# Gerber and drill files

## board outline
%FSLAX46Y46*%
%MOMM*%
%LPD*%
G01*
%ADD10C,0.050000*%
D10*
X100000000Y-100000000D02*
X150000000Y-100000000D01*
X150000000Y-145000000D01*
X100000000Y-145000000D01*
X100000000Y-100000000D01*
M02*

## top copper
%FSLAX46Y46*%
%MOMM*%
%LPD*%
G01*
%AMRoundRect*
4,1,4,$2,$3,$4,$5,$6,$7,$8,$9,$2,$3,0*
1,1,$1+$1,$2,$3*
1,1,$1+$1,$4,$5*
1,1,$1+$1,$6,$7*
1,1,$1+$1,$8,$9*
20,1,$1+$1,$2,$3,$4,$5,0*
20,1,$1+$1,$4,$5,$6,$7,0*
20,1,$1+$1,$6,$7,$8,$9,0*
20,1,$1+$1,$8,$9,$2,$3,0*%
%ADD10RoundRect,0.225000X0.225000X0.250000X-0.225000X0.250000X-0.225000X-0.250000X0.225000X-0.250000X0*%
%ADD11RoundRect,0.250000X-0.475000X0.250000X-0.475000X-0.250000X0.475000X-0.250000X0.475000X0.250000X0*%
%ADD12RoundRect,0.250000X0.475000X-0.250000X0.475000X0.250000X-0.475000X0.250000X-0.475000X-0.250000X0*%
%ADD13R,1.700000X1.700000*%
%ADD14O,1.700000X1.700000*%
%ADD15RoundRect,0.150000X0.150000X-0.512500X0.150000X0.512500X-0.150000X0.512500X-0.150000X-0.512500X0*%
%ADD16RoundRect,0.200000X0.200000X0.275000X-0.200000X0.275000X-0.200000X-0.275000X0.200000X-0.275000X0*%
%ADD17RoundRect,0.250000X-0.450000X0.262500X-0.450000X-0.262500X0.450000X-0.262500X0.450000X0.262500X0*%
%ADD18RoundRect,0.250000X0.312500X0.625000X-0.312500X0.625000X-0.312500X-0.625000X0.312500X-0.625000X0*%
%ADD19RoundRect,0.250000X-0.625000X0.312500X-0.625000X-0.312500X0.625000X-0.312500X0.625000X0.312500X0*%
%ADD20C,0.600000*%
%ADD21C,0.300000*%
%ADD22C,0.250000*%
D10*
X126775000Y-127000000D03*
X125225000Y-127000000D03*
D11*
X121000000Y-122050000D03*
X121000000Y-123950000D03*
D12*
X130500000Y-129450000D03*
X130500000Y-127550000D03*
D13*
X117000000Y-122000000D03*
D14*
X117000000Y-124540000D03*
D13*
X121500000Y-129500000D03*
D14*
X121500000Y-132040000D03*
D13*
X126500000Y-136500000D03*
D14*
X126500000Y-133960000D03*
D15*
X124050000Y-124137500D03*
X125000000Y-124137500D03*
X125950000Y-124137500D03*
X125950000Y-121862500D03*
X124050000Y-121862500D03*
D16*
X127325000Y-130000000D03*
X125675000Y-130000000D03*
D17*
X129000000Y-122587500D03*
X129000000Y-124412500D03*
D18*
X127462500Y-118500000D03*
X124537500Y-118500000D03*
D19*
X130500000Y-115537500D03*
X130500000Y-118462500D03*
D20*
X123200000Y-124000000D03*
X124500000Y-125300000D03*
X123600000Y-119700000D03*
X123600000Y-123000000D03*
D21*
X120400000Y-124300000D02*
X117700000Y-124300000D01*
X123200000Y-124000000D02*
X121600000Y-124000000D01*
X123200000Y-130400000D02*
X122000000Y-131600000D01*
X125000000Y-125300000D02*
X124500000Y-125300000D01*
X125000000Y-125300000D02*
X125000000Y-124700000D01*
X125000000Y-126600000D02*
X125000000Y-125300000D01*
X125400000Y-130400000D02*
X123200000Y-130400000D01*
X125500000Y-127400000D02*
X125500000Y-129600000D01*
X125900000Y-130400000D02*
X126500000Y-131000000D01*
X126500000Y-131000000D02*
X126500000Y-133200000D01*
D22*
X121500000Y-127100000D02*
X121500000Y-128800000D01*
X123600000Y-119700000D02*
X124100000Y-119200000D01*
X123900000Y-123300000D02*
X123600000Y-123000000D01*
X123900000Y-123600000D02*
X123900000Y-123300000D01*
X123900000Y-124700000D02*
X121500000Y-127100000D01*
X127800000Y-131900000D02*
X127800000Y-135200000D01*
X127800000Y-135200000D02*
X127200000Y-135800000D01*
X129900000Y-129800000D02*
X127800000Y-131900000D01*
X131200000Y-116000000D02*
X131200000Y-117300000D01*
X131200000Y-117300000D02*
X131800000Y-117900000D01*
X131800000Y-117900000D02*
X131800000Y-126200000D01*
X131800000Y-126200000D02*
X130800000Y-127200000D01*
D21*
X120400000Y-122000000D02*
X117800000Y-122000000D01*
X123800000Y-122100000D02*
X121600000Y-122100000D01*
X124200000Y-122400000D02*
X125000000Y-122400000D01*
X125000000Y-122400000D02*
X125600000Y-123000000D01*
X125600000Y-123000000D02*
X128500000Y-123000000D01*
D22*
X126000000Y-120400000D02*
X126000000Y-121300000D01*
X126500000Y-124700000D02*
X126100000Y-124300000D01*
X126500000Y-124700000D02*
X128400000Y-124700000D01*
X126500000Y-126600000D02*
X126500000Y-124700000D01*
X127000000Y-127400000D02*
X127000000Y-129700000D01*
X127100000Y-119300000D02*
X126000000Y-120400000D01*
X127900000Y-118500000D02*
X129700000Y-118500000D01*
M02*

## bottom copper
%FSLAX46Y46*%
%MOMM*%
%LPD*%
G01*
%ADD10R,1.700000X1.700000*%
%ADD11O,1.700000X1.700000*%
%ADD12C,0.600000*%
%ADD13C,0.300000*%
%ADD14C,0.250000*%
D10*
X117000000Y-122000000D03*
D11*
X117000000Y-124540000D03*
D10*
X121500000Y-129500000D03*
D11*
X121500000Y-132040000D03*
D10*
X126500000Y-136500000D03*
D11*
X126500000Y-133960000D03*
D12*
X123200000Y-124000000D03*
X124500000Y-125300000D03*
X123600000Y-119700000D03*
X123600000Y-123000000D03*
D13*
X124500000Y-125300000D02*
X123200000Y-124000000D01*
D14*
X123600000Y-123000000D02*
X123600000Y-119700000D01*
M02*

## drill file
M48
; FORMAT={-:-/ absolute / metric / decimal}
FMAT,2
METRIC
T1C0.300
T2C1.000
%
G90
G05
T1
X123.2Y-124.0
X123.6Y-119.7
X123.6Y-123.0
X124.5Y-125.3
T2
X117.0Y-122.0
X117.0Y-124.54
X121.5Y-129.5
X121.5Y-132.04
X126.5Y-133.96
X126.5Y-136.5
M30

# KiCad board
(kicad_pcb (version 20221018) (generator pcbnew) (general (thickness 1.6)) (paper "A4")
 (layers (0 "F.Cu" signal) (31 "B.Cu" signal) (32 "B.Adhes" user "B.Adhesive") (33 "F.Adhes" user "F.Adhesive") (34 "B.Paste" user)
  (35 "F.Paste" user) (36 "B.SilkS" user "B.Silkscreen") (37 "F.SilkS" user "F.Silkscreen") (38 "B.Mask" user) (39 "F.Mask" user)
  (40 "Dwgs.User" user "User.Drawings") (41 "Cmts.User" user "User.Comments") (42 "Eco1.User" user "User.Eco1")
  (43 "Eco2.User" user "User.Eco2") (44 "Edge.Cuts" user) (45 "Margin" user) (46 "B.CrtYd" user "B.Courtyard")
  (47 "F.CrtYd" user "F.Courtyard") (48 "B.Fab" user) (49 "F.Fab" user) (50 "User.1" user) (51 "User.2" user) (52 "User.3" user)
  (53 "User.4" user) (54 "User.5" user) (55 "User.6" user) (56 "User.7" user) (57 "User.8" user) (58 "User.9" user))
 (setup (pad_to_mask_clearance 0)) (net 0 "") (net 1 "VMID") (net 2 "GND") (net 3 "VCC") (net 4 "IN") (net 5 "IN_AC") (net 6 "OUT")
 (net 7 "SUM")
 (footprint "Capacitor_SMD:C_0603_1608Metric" (layer "F.Cu") (at 126 127 180)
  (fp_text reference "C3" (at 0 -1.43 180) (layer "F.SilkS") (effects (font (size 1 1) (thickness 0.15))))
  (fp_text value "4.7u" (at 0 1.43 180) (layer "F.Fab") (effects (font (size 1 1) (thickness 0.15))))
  (pad "1" smd roundrect (at -0.775 0 180) (size 0.9 0.95) (layers "F.Cu" "F.Paste" "F.Mask") (roundrect_rratio 0.25) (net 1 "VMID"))
  (pad "2" smd roundrect (at 0.775 0 180) (size 0.9 0.95) (layers "F.Cu" "F.Paste" "F.Mask") (roundrect_rratio 0.25) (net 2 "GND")))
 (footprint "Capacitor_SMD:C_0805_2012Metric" (layer "F.Cu") (at 121 123 -90)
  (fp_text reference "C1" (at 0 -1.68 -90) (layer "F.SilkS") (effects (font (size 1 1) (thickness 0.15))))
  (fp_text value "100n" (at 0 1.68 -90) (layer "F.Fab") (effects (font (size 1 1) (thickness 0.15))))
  (pad "1" smd roundrect (at -0.95 0 270) (size 1 1.45) (layers "F.Cu" "F.Paste" "F.Mask") (roundrect_rratio 0.25) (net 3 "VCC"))
  (pad "2" smd roundrect (at 0.95 0 270) (size 1 1.45) (layers "F.Cu" "F.Paste" "F.Mask") (roundrect_rratio 0.25) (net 2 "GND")))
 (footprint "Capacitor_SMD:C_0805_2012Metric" (layer "F.Cu") (at 130.5 128.5 90)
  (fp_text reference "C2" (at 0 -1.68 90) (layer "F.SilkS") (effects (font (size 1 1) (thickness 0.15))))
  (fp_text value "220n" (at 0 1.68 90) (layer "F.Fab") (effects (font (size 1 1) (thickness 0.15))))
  (pad "1" smd roundrect (at -0.95 0 90) (size 1 1.45) (layers "F.Cu" "F.Paste" "F.Mask") (roundrect_rratio 0.25) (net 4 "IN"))
  (pad "2" smd roundrect (at 0.95 0 90) (size 1 1.45) (layers "F.Cu" "F.Paste" "F.Mask") (roundrect_rratio 0.25) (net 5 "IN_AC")))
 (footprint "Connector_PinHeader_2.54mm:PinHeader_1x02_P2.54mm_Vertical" (layer "F.Cu") (at 117 122)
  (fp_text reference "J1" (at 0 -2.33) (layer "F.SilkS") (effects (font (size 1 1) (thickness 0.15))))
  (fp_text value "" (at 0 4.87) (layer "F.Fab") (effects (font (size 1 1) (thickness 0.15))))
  (pad "1" thru_hole rect (at 0 0) (size 1.7 1.7) (drill 1) (layers "*.Cu" "*.Mask") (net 3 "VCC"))
  (pad "2" thru_hole oval (at 0 2.54) (size 1.7 1.7) (drill 1) (layers "*.Cu" "*.Mask") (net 2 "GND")))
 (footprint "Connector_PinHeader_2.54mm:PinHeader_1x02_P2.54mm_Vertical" (layer "F.Cu") (at 121.5 129.5)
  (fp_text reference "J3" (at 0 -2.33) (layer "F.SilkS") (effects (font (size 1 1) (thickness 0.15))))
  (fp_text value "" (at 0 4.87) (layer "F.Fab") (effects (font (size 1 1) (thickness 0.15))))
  (pad "1" thru_hole rect (at 0 0) (size 1.7 1.7) (drill 1) (layers "*.Cu" "*.Mask") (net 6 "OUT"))
  (pad "2" thru_hole oval (at 0 2.54) (size 1.7 1.7) (drill 1) (layers "*.Cu" "*.Mask") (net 2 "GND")))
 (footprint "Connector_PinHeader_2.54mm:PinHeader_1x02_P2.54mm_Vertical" (layer "F.Cu") (at 126.5 136.5 180)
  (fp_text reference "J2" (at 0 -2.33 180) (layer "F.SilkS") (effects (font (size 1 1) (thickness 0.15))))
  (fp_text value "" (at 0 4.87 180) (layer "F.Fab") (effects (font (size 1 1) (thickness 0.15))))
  (pad "1" thru_hole rect (at 0 0 180) (size 1.7 1.7) (drill 1) (layers "*.Cu" "*.Mask") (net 4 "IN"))
  (pad "2" thru_hole oval (at 0 2.54 180) (size 1.7 1.7) (drill 1) (layers "*.Cu" "*.Mask") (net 2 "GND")))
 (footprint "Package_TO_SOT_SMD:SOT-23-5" (layer "F.Cu") (at 125 123 90)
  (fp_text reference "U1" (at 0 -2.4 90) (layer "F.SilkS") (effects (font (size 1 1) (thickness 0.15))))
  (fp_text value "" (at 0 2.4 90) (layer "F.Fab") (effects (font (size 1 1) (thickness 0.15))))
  (pad "1" smd roundrect (at -1.1375 -0.95 90) (size 1.325 0.6) (layers "F.Cu" "F.Paste" "F.Mask") (roundrect_rratio 0.25) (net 6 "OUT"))
  (pad "2" smd roundrect (at -1.1375 0 90) (size 1.325 0.6) (layers "F.Cu" "F.Paste" "F.Mask") (roundrect_rratio 0.25) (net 2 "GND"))
  (pad "3" smd roundrect (at -1.1375 0.95 90) (size 1.325 0.6) (layers "F.Cu" "F.Paste" "F.Mask") (roundrect_rratio 0.25) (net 1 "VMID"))
  (pad "4" smd roundrect (at 1.1375 0.95 90) (size 1.325 0.6) (layers "F.Cu" "F.Paste" "F.Mask") (roundrect_rratio 0.25) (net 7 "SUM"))
  (pad "5" smd roundrect (at 1.1375 -0.95 90) (size 1.325 0.6) (layers "F.Cu" "F.Paste" "F.Mask") (roundrect_rratio 0.25) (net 3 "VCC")))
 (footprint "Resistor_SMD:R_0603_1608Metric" (layer "F.Cu") (at 126.5 130 180)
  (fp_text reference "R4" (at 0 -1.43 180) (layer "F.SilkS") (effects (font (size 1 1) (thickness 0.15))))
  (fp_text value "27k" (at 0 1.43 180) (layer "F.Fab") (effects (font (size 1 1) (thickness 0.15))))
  (pad "1" smd roundrect (at -0.825 0 180) (size 0.8 0.95) (layers "F.Cu" "F.Paste" "F.Mask") (roundrect_rratio 0.25) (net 1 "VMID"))
  (pad "2" smd roundrect (at 0.825 0 180) (size 0.8 0.95) (layers "F.Cu" "F.Paste" "F.Mask") (roundrect_rratio 0.25) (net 2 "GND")))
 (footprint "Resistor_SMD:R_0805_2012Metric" (layer "F.Cu") (at 129 123.5 -90)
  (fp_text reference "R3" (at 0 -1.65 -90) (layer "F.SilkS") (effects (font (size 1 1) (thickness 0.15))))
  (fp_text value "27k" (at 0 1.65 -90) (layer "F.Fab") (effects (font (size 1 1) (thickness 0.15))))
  (pad "1" smd roundrect (at -0.9125 0 270) (size 1.025 1.4) (layers "F.Cu" "F.Paste" "F.Mask") (roundrect_rratio 0.243902) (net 3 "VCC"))
  (pad "2" smd roundrect (at 0.9125 0 270) (size 1.025 1.4) (layers "F.Cu" "F.Paste" "F.Mask") (roundrect_rratio 0.243902) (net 1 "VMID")))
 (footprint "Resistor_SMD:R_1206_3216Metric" (layer "F.Cu") (at 126 118.5 180)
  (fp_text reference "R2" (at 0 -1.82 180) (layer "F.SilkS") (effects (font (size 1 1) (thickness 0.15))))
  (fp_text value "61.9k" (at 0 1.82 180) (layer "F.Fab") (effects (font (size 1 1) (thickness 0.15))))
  (pad "1" smd roundrect (at -1.4625 0 180) (size 1.125 1.75) (layers "F.Cu" "F.Paste" "F.Mask") (roundrect_rratio 0.222222) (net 7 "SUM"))
  (pad "2" smd roundrect (at 1.4625 0 180) (size 1.125 1.75) (layers "F.Cu" "F.Paste" "F.Mask") (roundrect_rratio 0.222222) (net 6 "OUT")))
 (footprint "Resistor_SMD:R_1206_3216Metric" (layer "F.Cu") (at 130.5 117 -90)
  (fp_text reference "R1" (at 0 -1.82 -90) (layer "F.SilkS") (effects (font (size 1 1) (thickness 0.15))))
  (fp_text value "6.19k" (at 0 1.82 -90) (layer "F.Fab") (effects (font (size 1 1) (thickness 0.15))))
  (pad "1" smd roundrect (at -1.4625 0 270) (size 1.125 1.75) (layers "F.Cu" "F.Paste" "F.Mask") (roundrect_rratio 0.222222) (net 5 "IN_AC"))
  (pad "2" smd roundrect (at 1.4625 0 270) (size 1.125 1.75) (layers "F.Cu" "F.Paste" "F.Mask") (roundrect_rratio 0.222222) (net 7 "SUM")))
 (gr_rect (start 100 100) (end 150 145) (stroke (width 0.05) (type default)) (fill none) (layer "Edge.Cuts"))
 (segment (start 120.4 124.3) (end 117.7 124.3) (width 0.3) (layer "F.Cu") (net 2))
 (segment (start 123.2 124) (end 121.6 124) (width 0.3) (layer "F.Cu") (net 2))
 (segment (start 123.2 130.4) (end 122 131.6) (width 0.3) (layer "F.Cu") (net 2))
 (segment (start 125 125.3) (end 124.5 125.3) (width 0.3) (layer "F.Cu") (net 2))
 (segment (start 125 125.3) (end 125 124.7) (width 0.3) (layer "F.Cu") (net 2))
 (segment (start 125 126.6) (end 125 125.3) (width 0.3) (layer "F.Cu") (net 2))
 (segment (start 125.4 130.4) (end 123.2 130.4) (width 0.3) (layer "F.Cu") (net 2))
 (segment (start 125.5 127.4) (end 125.5 129.6) (width 0.3) (layer "F.Cu") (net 2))
 (segment (start 125.9 130.4) (end 126.5 131) (width 0.3) (layer "F.Cu") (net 2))
 (segment (start 126.5 131) (end 126.5 133.2) (width 0.3) (layer "F.Cu") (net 2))
 (via (at 123.2 124) (size 0.6) (drill 0.3) (layers "F.Cu" "B.Cu") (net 2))
 (via (at 124.5 125.3) (size 0.6) (drill 0.3) (layers "F.Cu" "B.Cu") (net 2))
 (segment (start 121.5 127.1) (end 121.5 128.8) (width 0.25) (layer "F.Cu") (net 6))
 (segment (start 123.6 119.7) (end 124.1 119.2) (width 0.25) (layer "F.Cu") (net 6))
 (segment (start 123.9 123.3) (end 123.6 123) (width 0.25) (layer "F.Cu") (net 6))
 (segment (start 123.9 123.6) (end 123.9 123.3) (width 0.25) (layer "F.Cu") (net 6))
 (segment (start 123.9 124.7) (end 121.5 127.1) (width 0.25) (layer "F.Cu") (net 6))
 (segment (start 124.5 125.3) (end 123.2 124) (width 0.3) (layer "B.Cu") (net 2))
 (segment (start 127.8 131.9) (end 127.8 135.2) (width 0.25) (layer "F.Cu") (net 4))
 (segment (start 127.8 135.2) (end 127.2 135.8) (width 0.25) (layer "F.Cu") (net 4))
 (segment (start 129.9 129.8) (end 127.8 131.9) (width 0.25) (layer "F.Cu") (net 4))
 (segment (start 131.2 116) (end 131.2 117.3) (width 0.25) (layer "F.Cu") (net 5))
 (segment (start 131.2 117.3) (end 131.8 117.9) (width 0.25) (layer "F.Cu") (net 5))
 (segment (start 131.8 117.9) (end 131.8 126.2) (width 0.25) (layer "F.Cu") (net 5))
 (segment (start 131.8 126.2) (end 130.8 127.2) (width 0.25) (layer "F.Cu") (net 5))
 (via (at 123.6 119.7) (size 0.6) (drill 0.3) (layers "F.Cu" "B.Cu") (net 6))
 (via (at 123.6 123) (size 0.6) (drill 0.3) (layers "F.Cu" "B.Cu") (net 6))
 (segment (start 120.4 122) (end 117.8 122) (width 0.3) (layer "F.Cu") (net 3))
 (segment (start 123.6 123) (end 123.6 119.7) (width 0.25) (layer "B.Cu") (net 6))
 (segment (start 123.8 122.1) (end 121.6 122.1) (width 0.3) (layer "F.Cu") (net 3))
 (segment (start 124.2 122.4) (end 125 122.4) (width 0.3) (layer "F.Cu") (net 3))
 (segment (start 125 122.4) (end 125.6 123) (width 0.3) (layer "F.Cu") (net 3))
 (segment (start 125.6 123) (end 128.5 123) (width 0.3) (layer "F.Cu") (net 3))
 (segment (start 126 120.4) (end 126 121.3) (width 0.25) (layer "F.Cu") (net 7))
 (segment (start 126.5 124.7) (end 126.1 124.3) (width 0.25) (layer "F.Cu") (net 1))
 (segment (start 126.5 124.7) (end 128.4 124.7) (width 0.25) (layer "F.Cu") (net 1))
 (segment (start 126.5 126.6) (end 126.5 124.7) (width 0.25) (layer "F.Cu") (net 1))
 (segment (start 127 127.4) (end 127 129.7) (width 0.25) (layer "F.Cu") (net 1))
 (segment (start 127.1 119.3) (end 126 120.4) (width 0.25) (layer "F.Cu") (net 7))
 (segment (start 127.9 118.5) (end 129.7 118.5) (width 0.25) (layer "F.Cu") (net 7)))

